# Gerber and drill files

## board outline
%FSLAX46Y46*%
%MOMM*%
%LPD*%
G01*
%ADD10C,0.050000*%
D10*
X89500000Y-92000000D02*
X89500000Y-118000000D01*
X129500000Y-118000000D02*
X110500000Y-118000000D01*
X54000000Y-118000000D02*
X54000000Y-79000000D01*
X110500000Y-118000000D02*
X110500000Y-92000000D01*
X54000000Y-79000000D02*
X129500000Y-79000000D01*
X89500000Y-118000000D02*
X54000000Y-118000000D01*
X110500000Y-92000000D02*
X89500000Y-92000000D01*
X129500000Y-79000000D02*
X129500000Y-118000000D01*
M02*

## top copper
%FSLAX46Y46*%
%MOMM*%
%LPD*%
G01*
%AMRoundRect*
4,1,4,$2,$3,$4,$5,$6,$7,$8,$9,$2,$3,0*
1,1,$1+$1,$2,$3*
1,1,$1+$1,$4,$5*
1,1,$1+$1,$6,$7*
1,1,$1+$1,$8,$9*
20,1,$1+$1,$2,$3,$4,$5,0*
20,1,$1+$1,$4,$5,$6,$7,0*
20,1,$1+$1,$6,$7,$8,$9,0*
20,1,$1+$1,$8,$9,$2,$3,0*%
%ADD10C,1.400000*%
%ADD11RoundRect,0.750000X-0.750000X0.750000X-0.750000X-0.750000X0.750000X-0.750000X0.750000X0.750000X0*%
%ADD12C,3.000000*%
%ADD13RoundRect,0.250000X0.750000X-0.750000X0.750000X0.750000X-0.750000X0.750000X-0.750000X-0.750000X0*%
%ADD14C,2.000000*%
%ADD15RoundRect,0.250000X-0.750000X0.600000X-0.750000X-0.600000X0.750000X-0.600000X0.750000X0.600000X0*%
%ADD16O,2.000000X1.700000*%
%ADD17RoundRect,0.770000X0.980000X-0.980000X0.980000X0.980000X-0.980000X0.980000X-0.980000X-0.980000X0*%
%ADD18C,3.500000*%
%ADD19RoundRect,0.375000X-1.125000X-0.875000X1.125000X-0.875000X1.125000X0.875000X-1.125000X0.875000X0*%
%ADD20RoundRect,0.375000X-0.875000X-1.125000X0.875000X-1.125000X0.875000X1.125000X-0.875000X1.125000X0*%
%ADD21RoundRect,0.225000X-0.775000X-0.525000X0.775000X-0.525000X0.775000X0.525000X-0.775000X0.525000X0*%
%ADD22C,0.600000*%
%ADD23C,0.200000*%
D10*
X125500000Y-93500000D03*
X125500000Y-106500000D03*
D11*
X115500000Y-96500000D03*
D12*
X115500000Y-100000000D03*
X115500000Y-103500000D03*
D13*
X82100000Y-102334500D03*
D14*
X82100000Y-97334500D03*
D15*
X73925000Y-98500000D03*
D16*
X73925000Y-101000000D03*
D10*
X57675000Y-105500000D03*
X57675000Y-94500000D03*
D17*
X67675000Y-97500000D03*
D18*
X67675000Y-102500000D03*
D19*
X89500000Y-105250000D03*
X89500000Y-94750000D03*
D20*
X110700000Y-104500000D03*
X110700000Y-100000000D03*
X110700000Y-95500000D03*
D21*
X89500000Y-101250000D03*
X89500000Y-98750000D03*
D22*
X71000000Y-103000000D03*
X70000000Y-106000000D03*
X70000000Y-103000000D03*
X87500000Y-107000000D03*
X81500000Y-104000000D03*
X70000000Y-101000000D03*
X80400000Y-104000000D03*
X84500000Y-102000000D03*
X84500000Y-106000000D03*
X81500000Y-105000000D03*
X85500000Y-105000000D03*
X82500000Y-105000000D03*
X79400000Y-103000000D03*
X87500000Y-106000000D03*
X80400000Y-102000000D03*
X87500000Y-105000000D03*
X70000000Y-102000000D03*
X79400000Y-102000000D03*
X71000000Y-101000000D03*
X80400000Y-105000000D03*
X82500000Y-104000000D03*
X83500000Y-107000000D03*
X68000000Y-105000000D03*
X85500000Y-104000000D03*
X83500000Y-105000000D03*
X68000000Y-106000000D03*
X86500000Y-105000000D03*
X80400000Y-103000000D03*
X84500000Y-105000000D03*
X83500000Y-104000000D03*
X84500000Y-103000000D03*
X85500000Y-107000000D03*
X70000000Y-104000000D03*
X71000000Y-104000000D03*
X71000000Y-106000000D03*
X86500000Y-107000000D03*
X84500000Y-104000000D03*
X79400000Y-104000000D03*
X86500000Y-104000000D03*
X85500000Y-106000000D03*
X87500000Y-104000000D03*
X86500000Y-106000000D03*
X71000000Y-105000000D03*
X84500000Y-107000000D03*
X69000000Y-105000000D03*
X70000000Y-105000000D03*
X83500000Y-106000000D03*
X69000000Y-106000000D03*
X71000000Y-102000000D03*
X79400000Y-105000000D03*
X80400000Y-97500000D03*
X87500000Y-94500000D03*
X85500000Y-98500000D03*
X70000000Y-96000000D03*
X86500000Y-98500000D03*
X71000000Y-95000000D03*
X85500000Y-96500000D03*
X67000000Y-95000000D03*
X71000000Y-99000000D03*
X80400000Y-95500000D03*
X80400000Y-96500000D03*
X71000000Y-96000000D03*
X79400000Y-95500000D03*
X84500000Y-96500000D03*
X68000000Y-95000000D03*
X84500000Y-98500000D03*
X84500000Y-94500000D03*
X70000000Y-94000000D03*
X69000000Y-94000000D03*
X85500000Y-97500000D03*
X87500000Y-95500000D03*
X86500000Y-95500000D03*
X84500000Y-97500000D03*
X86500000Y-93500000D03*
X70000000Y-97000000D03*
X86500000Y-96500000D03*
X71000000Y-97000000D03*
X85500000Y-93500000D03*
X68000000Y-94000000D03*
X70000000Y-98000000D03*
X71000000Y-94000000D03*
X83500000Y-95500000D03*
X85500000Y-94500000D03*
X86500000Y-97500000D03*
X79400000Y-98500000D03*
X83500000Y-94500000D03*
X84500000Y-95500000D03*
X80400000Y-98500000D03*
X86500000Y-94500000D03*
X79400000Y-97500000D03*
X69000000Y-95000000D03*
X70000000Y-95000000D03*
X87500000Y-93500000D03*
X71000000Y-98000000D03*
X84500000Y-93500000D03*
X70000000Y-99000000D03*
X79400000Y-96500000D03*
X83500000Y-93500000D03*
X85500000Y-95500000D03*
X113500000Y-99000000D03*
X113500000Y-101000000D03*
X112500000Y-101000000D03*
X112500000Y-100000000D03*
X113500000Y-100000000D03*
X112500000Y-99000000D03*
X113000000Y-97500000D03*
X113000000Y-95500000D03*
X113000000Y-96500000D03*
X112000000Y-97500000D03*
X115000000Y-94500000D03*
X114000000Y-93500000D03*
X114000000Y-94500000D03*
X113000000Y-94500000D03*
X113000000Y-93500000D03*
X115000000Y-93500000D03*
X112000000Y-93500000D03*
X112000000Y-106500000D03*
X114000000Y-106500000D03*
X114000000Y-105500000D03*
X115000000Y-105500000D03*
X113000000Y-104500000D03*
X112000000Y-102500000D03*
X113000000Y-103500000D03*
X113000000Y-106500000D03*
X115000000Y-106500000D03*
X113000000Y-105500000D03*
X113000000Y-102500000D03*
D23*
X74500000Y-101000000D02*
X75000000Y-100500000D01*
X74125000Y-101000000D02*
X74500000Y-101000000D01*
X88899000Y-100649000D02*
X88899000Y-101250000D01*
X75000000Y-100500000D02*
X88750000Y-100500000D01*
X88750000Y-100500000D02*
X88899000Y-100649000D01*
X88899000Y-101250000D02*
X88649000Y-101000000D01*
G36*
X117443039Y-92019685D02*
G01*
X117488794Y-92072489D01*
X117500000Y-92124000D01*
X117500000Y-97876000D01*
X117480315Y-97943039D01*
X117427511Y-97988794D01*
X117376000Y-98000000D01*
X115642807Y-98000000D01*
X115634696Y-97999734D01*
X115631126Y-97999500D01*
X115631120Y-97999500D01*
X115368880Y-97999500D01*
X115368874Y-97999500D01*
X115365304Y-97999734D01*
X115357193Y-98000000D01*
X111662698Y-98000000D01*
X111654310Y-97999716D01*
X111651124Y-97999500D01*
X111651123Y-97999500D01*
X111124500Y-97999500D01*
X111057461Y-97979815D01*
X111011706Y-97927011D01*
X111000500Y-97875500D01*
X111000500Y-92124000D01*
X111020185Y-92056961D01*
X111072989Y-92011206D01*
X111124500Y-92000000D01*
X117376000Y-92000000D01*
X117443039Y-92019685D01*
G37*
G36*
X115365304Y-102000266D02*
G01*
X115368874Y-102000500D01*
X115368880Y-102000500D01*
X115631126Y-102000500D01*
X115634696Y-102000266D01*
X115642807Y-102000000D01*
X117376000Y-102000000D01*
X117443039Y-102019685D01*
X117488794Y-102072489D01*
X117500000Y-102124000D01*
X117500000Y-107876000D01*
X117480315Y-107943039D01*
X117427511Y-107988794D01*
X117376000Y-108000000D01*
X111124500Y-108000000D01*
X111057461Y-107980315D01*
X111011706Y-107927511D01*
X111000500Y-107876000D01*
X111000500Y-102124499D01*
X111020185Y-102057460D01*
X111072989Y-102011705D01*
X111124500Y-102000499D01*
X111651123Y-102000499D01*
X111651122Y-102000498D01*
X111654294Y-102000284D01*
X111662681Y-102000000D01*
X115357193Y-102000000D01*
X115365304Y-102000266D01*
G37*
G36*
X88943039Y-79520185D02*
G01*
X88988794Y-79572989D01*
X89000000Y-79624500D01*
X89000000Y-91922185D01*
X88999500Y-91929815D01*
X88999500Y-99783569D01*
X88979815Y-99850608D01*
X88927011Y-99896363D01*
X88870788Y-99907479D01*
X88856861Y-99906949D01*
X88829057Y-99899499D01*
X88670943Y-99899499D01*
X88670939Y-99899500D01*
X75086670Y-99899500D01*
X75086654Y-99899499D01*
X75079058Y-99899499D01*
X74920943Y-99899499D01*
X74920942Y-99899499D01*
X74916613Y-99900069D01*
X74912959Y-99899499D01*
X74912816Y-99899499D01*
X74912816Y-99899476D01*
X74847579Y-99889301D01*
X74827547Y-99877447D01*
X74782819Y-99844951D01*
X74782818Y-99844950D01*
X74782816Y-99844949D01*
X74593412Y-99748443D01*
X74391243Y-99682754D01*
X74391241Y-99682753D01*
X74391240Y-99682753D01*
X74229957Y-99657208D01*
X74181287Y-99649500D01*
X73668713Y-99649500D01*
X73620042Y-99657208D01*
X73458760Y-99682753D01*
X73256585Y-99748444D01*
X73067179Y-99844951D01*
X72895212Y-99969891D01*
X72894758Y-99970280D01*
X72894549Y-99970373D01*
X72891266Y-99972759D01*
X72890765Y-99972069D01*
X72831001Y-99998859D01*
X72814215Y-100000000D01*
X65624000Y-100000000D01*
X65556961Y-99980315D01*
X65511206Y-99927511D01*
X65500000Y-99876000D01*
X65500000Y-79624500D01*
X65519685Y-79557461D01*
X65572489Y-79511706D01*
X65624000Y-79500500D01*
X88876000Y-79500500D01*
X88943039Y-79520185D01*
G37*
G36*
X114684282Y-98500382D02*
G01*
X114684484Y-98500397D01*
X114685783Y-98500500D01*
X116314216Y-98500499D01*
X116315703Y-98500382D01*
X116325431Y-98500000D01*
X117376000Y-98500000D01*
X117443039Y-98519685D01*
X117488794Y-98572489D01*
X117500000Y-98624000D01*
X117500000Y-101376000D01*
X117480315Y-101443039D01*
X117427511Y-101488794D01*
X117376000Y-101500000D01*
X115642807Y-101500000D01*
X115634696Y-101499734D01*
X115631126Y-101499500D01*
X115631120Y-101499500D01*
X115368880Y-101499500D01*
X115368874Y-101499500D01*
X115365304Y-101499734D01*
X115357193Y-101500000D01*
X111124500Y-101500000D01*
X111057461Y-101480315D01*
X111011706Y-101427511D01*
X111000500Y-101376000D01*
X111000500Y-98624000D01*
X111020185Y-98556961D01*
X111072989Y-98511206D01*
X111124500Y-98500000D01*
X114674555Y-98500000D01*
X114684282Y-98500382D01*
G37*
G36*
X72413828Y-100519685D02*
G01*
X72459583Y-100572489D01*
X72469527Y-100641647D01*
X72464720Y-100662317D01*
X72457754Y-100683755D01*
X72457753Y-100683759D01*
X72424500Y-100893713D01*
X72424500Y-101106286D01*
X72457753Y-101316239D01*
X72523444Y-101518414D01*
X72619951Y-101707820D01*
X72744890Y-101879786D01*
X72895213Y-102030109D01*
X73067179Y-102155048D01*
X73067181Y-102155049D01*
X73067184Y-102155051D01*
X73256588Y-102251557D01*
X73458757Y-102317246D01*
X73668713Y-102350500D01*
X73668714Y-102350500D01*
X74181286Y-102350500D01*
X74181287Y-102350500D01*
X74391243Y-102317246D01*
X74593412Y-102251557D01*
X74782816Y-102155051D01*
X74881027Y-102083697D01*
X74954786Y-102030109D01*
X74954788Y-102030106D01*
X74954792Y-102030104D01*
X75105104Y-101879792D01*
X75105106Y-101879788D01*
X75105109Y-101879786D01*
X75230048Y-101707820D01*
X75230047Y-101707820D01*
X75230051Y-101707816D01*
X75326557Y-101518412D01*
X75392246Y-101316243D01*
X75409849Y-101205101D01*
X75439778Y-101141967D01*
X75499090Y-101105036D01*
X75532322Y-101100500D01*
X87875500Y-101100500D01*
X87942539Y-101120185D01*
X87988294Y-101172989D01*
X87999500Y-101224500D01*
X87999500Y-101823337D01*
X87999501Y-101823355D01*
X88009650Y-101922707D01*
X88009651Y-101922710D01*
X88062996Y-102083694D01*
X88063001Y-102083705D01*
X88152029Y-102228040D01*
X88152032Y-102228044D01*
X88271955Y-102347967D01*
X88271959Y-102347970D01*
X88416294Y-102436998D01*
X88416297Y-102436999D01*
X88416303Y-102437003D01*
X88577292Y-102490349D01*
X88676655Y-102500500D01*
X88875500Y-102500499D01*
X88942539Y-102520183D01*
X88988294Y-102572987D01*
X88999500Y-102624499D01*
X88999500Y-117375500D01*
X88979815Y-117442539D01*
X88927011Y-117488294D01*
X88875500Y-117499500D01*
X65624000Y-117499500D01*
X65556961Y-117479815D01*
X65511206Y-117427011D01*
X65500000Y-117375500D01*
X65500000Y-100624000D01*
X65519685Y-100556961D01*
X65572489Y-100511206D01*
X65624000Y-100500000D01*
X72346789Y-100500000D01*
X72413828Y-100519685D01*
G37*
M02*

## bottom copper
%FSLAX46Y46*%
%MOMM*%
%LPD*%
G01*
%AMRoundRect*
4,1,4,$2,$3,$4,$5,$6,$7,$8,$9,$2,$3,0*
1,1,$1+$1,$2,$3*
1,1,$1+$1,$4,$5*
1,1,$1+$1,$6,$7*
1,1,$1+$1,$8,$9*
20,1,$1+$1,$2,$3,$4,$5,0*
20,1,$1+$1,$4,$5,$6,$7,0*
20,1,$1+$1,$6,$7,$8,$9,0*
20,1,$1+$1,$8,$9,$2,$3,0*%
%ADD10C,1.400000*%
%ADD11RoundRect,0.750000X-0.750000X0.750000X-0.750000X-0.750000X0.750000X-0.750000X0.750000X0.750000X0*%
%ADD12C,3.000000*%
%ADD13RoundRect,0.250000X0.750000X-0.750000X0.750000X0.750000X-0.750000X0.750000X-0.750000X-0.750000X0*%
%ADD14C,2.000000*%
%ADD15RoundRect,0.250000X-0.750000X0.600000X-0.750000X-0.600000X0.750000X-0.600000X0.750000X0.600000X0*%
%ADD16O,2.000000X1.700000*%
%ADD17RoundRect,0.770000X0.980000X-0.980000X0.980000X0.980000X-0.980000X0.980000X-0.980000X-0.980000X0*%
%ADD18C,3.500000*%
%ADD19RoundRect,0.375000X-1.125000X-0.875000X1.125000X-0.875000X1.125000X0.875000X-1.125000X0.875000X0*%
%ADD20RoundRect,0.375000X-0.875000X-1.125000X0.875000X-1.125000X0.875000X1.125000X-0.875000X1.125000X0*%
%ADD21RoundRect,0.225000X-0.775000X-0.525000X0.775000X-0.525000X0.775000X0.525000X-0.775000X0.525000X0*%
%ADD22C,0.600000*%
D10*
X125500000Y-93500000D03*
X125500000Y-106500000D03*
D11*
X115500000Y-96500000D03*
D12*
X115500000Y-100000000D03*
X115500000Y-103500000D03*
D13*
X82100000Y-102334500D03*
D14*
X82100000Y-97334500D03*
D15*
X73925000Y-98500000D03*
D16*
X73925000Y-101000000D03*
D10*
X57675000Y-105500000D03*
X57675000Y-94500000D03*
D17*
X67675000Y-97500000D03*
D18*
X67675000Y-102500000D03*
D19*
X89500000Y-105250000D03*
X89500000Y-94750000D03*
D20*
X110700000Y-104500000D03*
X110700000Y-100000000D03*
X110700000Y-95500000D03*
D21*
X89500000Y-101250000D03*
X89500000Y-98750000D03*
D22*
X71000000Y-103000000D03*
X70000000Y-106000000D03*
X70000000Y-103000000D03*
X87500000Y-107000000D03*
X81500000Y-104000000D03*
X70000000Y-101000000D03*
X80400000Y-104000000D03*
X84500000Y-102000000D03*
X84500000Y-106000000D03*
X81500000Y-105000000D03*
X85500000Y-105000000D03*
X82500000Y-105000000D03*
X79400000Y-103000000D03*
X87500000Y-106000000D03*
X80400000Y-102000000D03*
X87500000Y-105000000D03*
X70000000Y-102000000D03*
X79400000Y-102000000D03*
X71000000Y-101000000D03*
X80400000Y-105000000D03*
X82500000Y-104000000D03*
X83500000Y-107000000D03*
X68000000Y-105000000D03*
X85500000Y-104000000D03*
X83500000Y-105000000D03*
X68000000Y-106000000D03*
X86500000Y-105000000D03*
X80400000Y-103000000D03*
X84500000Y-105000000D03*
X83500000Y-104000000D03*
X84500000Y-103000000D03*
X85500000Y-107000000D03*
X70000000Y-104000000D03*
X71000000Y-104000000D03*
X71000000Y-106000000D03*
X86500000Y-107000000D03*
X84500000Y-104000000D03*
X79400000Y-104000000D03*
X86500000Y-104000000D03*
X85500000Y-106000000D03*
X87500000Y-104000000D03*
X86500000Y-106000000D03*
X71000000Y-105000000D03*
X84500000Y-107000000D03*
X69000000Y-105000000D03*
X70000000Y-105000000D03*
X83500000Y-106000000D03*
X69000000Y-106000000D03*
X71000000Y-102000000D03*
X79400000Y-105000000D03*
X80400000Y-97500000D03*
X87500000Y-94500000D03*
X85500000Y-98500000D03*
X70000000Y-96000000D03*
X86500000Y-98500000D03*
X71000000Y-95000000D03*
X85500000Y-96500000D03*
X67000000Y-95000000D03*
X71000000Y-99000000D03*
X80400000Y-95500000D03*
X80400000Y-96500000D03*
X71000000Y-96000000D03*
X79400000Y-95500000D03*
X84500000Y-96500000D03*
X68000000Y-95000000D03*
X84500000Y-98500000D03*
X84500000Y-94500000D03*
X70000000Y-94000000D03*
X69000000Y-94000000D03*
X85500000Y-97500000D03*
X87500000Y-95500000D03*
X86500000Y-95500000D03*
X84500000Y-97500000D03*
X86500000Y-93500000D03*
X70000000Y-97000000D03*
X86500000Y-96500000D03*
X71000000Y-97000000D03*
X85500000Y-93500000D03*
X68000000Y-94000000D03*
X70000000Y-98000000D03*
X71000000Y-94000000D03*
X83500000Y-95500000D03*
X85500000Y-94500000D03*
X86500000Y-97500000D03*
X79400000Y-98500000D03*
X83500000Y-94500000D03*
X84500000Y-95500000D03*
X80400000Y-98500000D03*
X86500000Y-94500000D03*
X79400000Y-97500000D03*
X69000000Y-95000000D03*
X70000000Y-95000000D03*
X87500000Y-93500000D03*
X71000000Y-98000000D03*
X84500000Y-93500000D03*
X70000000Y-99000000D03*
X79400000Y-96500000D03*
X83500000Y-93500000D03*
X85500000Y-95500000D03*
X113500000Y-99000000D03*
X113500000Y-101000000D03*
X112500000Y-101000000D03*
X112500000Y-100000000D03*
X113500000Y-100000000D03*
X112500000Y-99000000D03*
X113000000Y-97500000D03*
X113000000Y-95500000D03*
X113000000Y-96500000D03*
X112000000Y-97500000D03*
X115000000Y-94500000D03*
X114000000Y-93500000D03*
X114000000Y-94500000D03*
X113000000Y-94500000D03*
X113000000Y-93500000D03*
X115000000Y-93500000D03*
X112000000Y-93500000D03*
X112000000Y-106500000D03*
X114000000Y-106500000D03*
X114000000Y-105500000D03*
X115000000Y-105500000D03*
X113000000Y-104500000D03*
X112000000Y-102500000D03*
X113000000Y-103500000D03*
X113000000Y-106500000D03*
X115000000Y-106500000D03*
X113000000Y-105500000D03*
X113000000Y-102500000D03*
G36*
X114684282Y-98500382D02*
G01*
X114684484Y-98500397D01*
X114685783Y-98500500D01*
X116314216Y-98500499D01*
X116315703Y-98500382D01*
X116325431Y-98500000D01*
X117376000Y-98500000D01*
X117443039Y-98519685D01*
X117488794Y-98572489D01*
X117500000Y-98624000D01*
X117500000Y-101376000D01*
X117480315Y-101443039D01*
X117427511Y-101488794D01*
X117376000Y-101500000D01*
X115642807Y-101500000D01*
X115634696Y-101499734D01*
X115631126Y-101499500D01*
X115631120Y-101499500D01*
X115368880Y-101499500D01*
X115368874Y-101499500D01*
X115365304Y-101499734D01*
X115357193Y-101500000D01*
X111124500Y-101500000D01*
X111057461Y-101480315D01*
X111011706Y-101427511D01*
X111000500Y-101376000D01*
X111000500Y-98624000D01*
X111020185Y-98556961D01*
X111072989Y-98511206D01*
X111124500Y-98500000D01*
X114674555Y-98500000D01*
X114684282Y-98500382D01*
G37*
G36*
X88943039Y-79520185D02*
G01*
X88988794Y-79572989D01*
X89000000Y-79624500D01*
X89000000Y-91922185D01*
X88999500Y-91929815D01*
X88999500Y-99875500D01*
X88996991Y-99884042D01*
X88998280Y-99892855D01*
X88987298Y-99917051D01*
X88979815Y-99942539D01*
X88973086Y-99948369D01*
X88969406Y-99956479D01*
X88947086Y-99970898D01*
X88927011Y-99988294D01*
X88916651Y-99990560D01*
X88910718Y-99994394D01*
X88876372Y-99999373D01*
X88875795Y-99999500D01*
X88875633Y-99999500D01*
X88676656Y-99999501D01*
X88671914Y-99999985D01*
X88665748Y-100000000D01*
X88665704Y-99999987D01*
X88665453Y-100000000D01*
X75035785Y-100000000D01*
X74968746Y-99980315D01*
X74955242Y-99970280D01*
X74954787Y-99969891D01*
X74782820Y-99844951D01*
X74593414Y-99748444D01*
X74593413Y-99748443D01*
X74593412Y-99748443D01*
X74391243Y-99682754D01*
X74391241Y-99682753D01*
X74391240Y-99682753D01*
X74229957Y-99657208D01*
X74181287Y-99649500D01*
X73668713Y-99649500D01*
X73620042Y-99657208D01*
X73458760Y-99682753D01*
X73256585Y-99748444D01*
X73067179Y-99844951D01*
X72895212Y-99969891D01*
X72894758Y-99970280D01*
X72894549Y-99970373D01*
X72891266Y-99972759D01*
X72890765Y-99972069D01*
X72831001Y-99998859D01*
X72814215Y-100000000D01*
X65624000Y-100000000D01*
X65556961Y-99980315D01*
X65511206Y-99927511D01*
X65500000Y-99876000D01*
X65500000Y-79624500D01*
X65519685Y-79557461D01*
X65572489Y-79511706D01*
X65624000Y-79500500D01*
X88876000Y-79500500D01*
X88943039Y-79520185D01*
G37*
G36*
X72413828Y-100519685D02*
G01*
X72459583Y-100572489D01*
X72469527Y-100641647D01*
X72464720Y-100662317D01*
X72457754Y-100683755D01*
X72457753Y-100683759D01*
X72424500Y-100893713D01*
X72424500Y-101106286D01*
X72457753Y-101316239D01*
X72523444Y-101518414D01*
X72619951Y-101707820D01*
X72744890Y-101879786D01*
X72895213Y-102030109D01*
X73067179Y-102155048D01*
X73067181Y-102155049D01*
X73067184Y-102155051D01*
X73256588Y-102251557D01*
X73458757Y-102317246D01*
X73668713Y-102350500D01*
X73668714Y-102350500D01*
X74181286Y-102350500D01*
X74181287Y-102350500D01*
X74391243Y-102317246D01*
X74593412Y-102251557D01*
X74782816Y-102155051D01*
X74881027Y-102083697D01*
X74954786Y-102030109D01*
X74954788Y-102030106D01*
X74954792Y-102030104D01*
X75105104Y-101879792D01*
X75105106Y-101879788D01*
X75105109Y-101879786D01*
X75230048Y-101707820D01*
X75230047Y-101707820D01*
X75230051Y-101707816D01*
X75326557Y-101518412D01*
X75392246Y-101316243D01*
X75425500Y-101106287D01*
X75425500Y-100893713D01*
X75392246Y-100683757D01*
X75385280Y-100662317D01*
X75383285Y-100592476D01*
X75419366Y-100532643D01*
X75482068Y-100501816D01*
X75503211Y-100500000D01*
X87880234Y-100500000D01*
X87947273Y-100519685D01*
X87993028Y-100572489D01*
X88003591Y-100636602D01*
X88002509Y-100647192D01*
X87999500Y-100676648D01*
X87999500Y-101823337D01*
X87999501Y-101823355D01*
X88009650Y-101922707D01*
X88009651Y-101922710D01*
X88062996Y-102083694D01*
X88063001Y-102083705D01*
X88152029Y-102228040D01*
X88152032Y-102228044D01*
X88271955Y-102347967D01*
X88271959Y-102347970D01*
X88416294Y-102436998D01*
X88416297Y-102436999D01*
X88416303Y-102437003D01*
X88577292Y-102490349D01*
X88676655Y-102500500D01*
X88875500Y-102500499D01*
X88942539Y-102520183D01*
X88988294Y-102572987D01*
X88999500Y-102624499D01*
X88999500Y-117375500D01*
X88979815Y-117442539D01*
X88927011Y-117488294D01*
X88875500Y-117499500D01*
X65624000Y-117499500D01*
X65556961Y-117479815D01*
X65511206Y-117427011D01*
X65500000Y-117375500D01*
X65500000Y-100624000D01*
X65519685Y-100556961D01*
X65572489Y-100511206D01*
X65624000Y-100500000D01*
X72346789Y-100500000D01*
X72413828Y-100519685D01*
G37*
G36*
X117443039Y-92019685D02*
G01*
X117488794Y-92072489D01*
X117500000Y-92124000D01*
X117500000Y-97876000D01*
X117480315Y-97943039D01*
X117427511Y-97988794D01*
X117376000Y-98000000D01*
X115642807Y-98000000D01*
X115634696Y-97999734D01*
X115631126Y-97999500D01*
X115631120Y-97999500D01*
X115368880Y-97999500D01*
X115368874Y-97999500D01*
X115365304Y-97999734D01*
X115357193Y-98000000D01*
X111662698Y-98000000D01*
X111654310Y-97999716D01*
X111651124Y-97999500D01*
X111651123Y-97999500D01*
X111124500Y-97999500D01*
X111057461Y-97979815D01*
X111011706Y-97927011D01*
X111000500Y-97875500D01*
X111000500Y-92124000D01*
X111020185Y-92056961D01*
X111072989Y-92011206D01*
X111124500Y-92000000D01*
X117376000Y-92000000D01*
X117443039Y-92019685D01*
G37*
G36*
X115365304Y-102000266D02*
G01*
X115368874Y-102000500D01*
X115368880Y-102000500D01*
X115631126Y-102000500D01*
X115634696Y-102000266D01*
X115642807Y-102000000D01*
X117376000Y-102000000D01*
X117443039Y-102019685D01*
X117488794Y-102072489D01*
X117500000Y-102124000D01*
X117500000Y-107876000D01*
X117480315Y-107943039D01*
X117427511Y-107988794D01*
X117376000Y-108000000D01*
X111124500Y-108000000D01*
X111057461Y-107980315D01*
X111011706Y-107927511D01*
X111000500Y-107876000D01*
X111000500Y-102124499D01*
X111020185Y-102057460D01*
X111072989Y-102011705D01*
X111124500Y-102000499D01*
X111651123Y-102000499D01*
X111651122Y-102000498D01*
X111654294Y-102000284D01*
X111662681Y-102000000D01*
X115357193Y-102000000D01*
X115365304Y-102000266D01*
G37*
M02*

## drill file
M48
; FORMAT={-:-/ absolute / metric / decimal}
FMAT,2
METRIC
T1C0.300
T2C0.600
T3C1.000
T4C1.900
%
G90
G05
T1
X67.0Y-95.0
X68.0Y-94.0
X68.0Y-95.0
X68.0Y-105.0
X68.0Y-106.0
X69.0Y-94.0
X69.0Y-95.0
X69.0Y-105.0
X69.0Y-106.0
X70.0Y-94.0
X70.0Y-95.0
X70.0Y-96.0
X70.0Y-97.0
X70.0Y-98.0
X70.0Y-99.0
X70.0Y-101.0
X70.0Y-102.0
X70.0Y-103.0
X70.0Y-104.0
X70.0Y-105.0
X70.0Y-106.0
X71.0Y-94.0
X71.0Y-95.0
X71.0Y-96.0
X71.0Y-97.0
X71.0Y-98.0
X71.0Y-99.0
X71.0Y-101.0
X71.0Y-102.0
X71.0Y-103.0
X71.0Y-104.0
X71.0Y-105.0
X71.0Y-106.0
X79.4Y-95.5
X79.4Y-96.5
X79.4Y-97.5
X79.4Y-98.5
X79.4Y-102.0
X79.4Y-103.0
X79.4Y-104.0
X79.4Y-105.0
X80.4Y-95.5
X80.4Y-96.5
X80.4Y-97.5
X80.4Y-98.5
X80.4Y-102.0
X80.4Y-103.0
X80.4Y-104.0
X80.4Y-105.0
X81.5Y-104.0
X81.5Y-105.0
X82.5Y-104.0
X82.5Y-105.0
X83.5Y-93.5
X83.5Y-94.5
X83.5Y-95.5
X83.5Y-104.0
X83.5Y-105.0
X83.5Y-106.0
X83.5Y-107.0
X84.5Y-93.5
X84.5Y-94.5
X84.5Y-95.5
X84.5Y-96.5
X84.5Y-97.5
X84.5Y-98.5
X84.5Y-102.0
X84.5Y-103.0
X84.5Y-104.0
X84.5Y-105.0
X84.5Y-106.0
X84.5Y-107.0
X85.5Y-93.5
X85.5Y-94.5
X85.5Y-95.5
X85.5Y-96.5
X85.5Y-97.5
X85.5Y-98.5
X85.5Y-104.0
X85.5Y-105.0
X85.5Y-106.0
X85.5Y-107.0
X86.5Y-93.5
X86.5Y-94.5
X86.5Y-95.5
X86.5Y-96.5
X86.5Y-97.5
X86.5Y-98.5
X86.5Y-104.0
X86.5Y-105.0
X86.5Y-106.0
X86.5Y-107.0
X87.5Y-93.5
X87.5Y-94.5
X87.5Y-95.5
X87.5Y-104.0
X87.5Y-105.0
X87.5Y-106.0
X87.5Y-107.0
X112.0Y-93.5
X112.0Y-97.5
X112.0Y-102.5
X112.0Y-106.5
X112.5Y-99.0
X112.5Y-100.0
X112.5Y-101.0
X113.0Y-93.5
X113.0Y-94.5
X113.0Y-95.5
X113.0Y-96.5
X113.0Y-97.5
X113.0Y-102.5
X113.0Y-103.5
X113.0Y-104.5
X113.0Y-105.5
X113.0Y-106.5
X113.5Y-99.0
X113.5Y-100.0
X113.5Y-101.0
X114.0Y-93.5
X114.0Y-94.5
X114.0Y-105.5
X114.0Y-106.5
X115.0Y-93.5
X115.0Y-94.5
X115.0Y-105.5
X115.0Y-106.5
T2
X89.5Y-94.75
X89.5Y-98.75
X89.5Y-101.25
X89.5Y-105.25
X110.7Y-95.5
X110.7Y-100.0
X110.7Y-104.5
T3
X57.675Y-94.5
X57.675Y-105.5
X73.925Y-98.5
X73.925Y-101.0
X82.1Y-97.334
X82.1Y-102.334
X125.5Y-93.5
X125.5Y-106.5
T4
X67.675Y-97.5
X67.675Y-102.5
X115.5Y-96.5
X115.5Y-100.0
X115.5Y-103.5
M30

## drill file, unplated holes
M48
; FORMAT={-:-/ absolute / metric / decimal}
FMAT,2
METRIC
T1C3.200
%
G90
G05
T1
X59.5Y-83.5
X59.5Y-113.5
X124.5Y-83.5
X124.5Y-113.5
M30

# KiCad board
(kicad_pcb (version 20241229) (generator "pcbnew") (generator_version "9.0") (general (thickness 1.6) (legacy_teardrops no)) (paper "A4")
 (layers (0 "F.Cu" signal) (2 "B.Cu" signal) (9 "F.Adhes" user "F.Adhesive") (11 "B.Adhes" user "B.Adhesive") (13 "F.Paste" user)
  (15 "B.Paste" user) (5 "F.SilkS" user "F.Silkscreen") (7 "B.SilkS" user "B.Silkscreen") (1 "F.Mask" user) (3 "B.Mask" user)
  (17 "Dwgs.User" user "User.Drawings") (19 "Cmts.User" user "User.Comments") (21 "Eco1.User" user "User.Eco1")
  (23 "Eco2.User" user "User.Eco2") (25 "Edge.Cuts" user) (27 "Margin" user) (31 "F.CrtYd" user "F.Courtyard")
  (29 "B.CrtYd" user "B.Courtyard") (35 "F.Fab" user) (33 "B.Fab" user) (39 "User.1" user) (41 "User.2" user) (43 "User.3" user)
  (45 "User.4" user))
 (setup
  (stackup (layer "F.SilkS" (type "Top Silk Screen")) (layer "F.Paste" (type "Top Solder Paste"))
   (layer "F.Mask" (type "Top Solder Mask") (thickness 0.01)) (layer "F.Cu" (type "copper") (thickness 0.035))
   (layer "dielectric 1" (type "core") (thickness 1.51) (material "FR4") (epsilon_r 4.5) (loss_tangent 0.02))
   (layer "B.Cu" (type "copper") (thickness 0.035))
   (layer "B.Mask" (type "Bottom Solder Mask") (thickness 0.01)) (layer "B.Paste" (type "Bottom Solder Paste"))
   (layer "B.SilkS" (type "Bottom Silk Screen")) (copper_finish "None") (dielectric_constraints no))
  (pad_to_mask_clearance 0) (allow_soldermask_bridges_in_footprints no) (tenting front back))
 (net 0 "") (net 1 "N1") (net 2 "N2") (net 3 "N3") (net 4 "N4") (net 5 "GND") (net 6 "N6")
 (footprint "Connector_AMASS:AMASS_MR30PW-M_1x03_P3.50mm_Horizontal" (layer "F.Cu") (at 115.5 96.5 -90)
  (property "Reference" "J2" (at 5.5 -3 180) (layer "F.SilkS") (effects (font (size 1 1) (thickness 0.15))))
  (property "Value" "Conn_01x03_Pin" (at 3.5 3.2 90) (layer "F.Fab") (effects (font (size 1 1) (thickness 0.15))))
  (pad "" thru_hole circle (at -3 -10 270) (size 1.4 1.4) (drill 1) (layers "*.Cu" "*.Mask") (remove_unused_layers no))
  (pad "" thru_hole circle (at 10 -10 270) (size 1.4 1.4) (drill 1) (layers "*.Cu" "*.Mask") (remove_unused_layers no))
  (pad "1" thru_hole roundrect (at 0 0 270) (size 3 3) (drill 1.9) (layers "*.Cu" "*.Mask") (remove_unused_layers no)
   (roundrect_rratio 0.25) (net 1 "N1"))
  (pad "2" thru_hole circle (at 3.5 0 270) (size 3 3) (drill 1.9) (layers "*.Cu" "*.Mask") (remove_unused_layers no) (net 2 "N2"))
  (pad "3" thru_hole circle (at 7 0 270) (size 3 3) (drill 1.9) (layers "*.Cu" "*.Mask") (remove_unused_layers no) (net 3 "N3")))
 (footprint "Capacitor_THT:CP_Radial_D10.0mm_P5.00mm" (layer "F.Cu") (at 82.1 102.3345 90)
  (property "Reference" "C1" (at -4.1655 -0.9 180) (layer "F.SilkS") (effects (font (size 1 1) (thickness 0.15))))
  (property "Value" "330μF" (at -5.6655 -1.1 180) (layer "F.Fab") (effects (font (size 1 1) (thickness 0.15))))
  (pad "1" thru_hole roundrect (at 0 0 90) (size 2 2) (drill 1) (layers "*.Cu" "*.Mask") (remove_unused_layers no) (roundrect_rratio 0.125)
   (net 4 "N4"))
  (pad "2" thru_hole circle (at 5 0 90) (size 2 2) (drill 1) (layers "*.Cu" "*.Mask") (remove_unused_layers no) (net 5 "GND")))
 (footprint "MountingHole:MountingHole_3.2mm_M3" (layer "F.Cu") (at 59.5 83.5)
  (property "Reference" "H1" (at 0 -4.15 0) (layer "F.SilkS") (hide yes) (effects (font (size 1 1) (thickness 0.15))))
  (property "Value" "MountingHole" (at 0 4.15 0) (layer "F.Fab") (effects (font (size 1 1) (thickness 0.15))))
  (pad "" np_thru_hole circle (at 0 0) (size 3.2 3.2) (drill 3.2) (layers "*.Cu" "*.Mask")))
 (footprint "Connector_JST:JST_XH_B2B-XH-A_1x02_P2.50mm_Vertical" (layer "F.Cu") (at 73.925 98.5 -90)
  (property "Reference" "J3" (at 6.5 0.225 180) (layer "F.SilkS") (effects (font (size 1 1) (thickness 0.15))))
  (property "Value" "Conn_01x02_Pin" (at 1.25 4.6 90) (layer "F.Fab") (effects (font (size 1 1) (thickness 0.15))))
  (pad "1" thru_hole roundrect (at 0 0 270) (size 1.7 2) (drill 1) (layers "*.Cu" "*.Mask") (remove_unused_layers no)
   (roundrect_rratio 0.147059) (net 5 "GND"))
  (pad "2" thru_hole oval (at 2.5 0 270) (size 1.7 2) (drill 1) (layers "*.Cu" "*.Mask") (remove_unused_layers no) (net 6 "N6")))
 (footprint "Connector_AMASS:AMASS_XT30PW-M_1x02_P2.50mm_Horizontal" (layer "F.Cu") (at 67.675 97.5 90)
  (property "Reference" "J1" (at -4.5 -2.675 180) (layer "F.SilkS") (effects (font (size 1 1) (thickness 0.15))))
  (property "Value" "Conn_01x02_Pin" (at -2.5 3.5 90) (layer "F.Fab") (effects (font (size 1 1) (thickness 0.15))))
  (pad "" thru_hole circle (at -8 -10 90) (size 1.4 1.4) (drill 1) (layers "*.Cu" "*.Mask") (remove_unused_layers no))
  (pad "" thru_hole circle (at 3 -10 90) (size 1.4 1.4) (drill 1) (layers "*.Cu" "*.Mask") (remove_unused_layers no))
  (pad "1" thru_hole roundrect (at 0 0 90) (size 3.5 3.5) (drill 1.9) (layers "*.Cu" "*.Mask") (remove_unused_layers no)
   (roundrect_rratio 0.22) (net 5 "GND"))
  (pad "2" thru_hole circle (at -5 0 90) (size 3.5 3.5) (drill 1.9) (layers "*.Cu" "*.Mask") (remove_unused_layers no) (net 4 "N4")))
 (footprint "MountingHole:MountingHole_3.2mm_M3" (layer "F.Cu") (at 124.5 113.5)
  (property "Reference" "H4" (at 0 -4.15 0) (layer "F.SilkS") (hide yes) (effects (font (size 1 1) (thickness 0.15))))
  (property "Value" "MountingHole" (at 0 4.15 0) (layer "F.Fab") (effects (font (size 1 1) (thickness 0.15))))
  (pad "" np_thru_hole circle (at 0 0) (size 3.2 3.2) (drill 3.2) (layers "*.Cu" "*.Mask")))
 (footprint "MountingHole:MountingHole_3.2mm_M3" (layer "F.Cu") (at 124.5 83.5)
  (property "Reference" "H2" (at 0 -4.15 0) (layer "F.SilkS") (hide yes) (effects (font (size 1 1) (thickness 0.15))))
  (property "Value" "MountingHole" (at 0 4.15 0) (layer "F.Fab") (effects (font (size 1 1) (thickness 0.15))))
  (pad "" np_thru_hole circle (at 0 0) (size 3.2 3.2) (drill 3.2) (layers "*.Cu" "*.Mask")))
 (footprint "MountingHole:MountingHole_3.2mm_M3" (layer "F.Cu") (at 59.5 113.5)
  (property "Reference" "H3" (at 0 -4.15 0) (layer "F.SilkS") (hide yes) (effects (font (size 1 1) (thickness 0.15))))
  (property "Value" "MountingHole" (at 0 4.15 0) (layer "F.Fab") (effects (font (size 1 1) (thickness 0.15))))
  (pad "" np_thru_hole circle (at 0 0) (size 3.2 3.2) (drill 3.2) (layers "*.Cu" "*.Mask")))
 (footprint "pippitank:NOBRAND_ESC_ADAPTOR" (layer "B.Cu") (at 100 100)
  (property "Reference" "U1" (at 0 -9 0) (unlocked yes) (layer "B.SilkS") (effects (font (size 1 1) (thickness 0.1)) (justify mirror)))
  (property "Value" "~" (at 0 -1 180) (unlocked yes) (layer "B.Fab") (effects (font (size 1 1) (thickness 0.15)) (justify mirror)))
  (pad "1" thru_hole roundrect (at -10.5 5.25) (size 3 2.5) (drill 0.6) (layers "*.Cu" "*.Mask") (remove_unused_layers no)
   (roundrect_rratio 0.15) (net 4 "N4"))
  (pad "2" thru_hole roundrect (at -10.5 -5.25) (size 3 2.5) (drill 0.6) (layers "*.Cu" "*.Mask") (remove_unused_layers no)
   (roundrect_rratio 0.15) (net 5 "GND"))
  (pad "3" thru_hole roundrect (at 10.7 4.5) (size 2.5 3) (drill 0.6) (layers "*.Cu" "*.Mask") (remove_unused_layers no)
   (roundrect_rratio 0.15) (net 3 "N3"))
  (pad "4" thru_hole roundrect (at 10.7 0) (size 2.5 3) (drill 0.6) (layers "*.Cu" "*.Mask") (remove_unused_layers no)
   (roundrect_rratio 0.15) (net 2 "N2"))
  (pad "5" thru_hole roundrect (at 10.7 -4.5) (size 2.5 3) (drill 0.6) (layers "*.Cu" "*.Mask") (remove_unused_layers no)
   (roundrect_rratio 0.15) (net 1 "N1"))
  (pad "6" thru_hole roundrect (at -10.5 1.25) (size 2 1.5) (drill 0.6) (layers "*.Cu" "*.Mask") (remove_unused_layers no)
   (roundrect_rratio 0.15) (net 6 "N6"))
  (pad "7" thru_hole roundrect (at -10.5 -1.25) (size 2 1.5) (drill 0.6) (layers "*.Cu" "*.Mask") (remove_unused_layers no)
   (roundrect_rratio 0.15) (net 5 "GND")))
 (gr_line (start 89.5 92) (end 89.5 118) (stroke (width 0.05) (type default)) (layer "Edge.Cuts"))
 (gr_line (start 129.5 118) (end 110.5 118) (stroke (width 0.05) (type solid)) (layer "Edge.Cuts"))
 (gr_line (start 54 118) (end 54 79) (stroke (width 0.05) (type solid)) (layer "Edge.Cuts"))
 (gr_line (start 110.5 118) (end 110.5 92) (stroke (width 0.05) (type default)) (layer "Edge.Cuts"))
 (gr_line (start 54 79) (end 129.5 79) (stroke (width 0.05) (type solid)) (layer "Edge.Cuts"))
 (gr_line (start 89.5 118) (end 54 118) (stroke (width 0.05) (type solid)) (layer "Edge.Cuts"))
 (gr_line (start 110.5 92) (end 89.5 92) (stroke (width 0.05) (type default)) (layer "Edge.Cuts"))
 (gr_line (start 129.5 79) (end 129.5 118) (stroke (width 0.05) (type default)) (layer "Edge.Cuts"))
 (via (at 71 103) (size 0.6) (drill 0.3) (layers "F.Cu" "B.Cu") (free yes) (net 4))
 (via (at 70 106) (size 0.6) (drill 0.3) (layers "F.Cu" "B.Cu") (free yes) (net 4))
 (via (at 70 103) (size 0.6) (drill 0.3) (layers "F.Cu" "B.Cu") (free yes) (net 4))
 (via (at 87.5 107) (size 0.6) (drill 0.3) (layers "F.Cu" "B.Cu") (free yes) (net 4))
 (via (at 81.5 104) (size 0.6) (drill 0.3) (layers "F.Cu" "B.Cu") (free yes) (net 4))
 (via (at 70 101) (size 0.6) (drill 0.3) (layers "F.Cu" "B.Cu") (free yes) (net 4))
 (via (at 80.4 104) (size 0.6) (drill 0.3) (layers "F.Cu" "B.Cu") (free yes) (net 4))
 (via (at 84.5 102) (size 0.6) (drill 0.3) (layers "F.Cu" "B.Cu") (free yes) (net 4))
 (via (at 84.5 106) (size 0.6) (drill 0.3) (layers "F.Cu" "B.Cu") (free yes) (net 4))
 (via (at 81.5 105) (size 0.6) (drill 0.3) (layers "F.Cu" "B.Cu") (free yes) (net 4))
 (via (at 85.5 105) (size 0.6) (drill 0.3) (layers "F.Cu" "B.Cu") (free yes) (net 4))
 (via (at 82.5 105) (size 0.6) (drill 0.3) (layers "F.Cu" "B.Cu") (free yes) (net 4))
 (via (at 79.4 103) (size 0.6) (drill 0.3) (layers "F.Cu" "B.Cu") (free yes) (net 4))
 (via (at 87.5 106) (size 0.6) (drill 0.3) (layers "F.Cu" "B.Cu") (free yes) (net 4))
 (via (at 80.4 102) (size 0.6) (drill 0.3) (layers "F.Cu" "B.Cu") (free yes) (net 4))
 (via (at 87.5 105) (size 0.6) (drill 0.3) (layers "F.Cu" "B.Cu") (free yes) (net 4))
 (via (at 70 102) (size 0.6) (drill 0.3) (layers "F.Cu" "B.Cu") (free yes) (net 4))
 (via (at 79.4 102) (size 0.6) (drill 0.3) (layers "F.Cu" "B.Cu") (free yes) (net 4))
 (via (at 71 101) (size 0.6) (drill 0.3) (layers "F.Cu" "B.Cu") (free yes) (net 4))
 (via (at 80.4 105) (size 0.6) (drill 0.3) (layers "F.Cu" "B.Cu") (free yes) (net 4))
 (via (at 82.5 104) (size 0.6) (drill 0.3) (layers "F.Cu" "B.Cu") (free yes) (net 4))
 (via (at 83.5 107) (size 0.6) (drill 0.3) (layers "F.Cu" "B.Cu") (free yes) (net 4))
 (via (at 68 105) (size 0.6) (drill 0.3) (layers "F.Cu" "B.Cu") (free yes) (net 4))
 (via (at 85.5 104) (size 0.6) (drill 0.3) (layers "F.Cu" "B.Cu") (free yes) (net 4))
 (via (at 83.5 105) (size 0.6) (drill 0.3) (layers "F.Cu" "B.Cu") (free yes) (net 4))
 (via (at 68 106) (size 0.6) (drill 0.3) (layers "F.Cu" "B.Cu") (free yes) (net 4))
 (via (at 86.5 105) (size 0.6) (drill 0.3) (layers "F.Cu" "B.Cu") (free yes) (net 4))
 (via (at 80.4 103) (size 0.6) (drill 0.3) (layers "F.Cu" "B.Cu") (free yes) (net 4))
 (via (at 84.5 105) (size 0.6) (drill 0.3) (layers "F.Cu" "B.Cu") (free yes) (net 4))
 (via (at 83.5 104) (size 0.6) (drill 0.3) (layers "F.Cu" "B.Cu") (free yes) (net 4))
 (via (at 84.5 103) (size 0.6) (drill 0.3) (layers "F.Cu" "B.Cu") (free yes) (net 4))
 (via (at 85.5 107) (size 0.6) (drill 0.3) (layers "F.Cu" "B.Cu") (free yes) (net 4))
 (via (at 70 104) (size 0.6) (drill 0.3) (layers "F.Cu" "B.Cu") (free yes) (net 4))
 (via (at 71 104) (size 0.6) (drill 0.3) (layers "F.Cu" "B.Cu") (free yes) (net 4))
 (via (at 71 106) (size 0.6) (drill 0.3) (layers "F.Cu" "B.Cu") (free yes) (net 4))
 (via (at 86.5 107) (size 0.6) (drill 0.3) (layers "F.Cu" "B.Cu") (free yes) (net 4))
 (via (at 84.5 104) (size 0.6) (drill 0.3) (layers "F.Cu" "B.Cu") (free yes) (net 4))
 (via (at 79.4 104) (size 0.6) (drill 0.3) (layers "F.Cu" "B.Cu") (free yes) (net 4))
 (via (at 86.5 104) (size 0.6) (drill 0.3) (layers "F.Cu" "B.Cu") (free yes) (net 4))
 (via (at 85.5 106) (size 0.6) (drill 0.3) (layers "F.Cu" "B.Cu") (free yes) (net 4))
 (via (at 87.5 104) (size 0.6) (drill 0.3) (layers "F.Cu" "B.Cu") (free yes) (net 4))
 (via (at 86.5 106) (size 0.6) (drill 0.3) (layers "F.Cu" "B.Cu") (free yes) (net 4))
 (via (at 71 105) (size 0.6) (drill 0.3) (layers "F.Cu" "B.Cu") (free yes) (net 4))
 (via (at 84.5 107) (size 0.6) (drill 0.3) (layers "F.Cu" "B.Cu") (free yes) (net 4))
 (via (at 69 105) (size 0.6) (drill 0.3) (layers "F.Cu" "B.Cu") (free yes) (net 4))
 (via (at 70 105) (size 0.6) (drill 0.3) (layers "F.Cu" "B.Cu") (free yes) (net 4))
 (via (at 83.5 106) (size 0.6) (drill 0.3) (layers "F.Cu" "B.Cu") (free yes) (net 4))
 (via (at 69 106) (size 0.6) (drill 0.3) (layers "F.Cu" "B.Cu") (free yes) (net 4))
 (via (at 71 102) (size 0.6) (drill 0.3) (layers "F.Cu" "B.Cu") (free yes) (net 4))
 (via (at 79.4 105) (size 0.6) (drill 0.3) (layers "F.Cu" "B.Cu") (free yes) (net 4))
 (via (at 80.4 97.5) (size 0.6) (drill 0.3) (layers "F.Cu" "B.Cu") (free yes) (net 5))
 (via (at 87.5 94.5) (size 0.6) (drill 0.3) (layers "F.Cu" "B.Cu") (free yes) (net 5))
 (via (at 85.5 98.5) (size 0.6) (drill 0.3) (layers "F.Cu" "B.Cu") (free yes) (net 5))
 (via (at 70 96) (size 0.6) (drill 0.3) (layers "F.Cu" "B.Cu") (free yes) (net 5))
 (via (at 86.5 98.5) (size 0.6) (drill 0.3) (layers "F.Cu" "B.Cu") (free yes) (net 5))
 (via (at 71 95) (size 0.6) (drill 0.3) (layers "F.Cu" "B.Cu") (free yes) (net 5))
 (via (at 85.5 96.5) (size 0.6) (drill 0.3) (layers "F.Cu" "B.Cu") (free yes) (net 5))
 (via (at 67 95) (size 0.6) (drill 0.3) (layers "F.Cu" "B.Cu") (free yes) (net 5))
 (via (at 71 99) (size 0.6) (drill 0.3) (layers "F.Cu" "B.Cu") (free yes) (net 5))
 (via (at 80.4 95.5) (size 0.6) (drill 0.3) (layers "F.Cu" "B.Cu") (free yes) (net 5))
 (via (at 80.4 96.5) (size 0.6) (drill 0.3) (layers "F.Cu" "B.Cu") (free yes) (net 5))
 (via (at 71 96) (size 0.6) (drill 0.3) (layers "F.Cu" "B.Cu") (free yes) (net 5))
 (via (at 79.4 95.5) (size 0.6) (drill 0.3) (layers "F.Cu" "B.Cu") (free yes) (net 5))
 (via (at 84.5 96.5) (size 0.6) (drill 0.3) (layers "F.Cu" "B.Cu") (free yes) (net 5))
 (via (at 68 95) (size 0.6) (drill 0.3) (layers "F.Cu" "B.Cu") (free yes) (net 5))
 (via (at 84.5 98.5) (size 0.6) (drill 0.3) (layers "F.Cu" "B.Cu") (free yes) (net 5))
 (via (at 84.5 94.5) (size 0.6) (drill 0.3) (layers "F.Cu" "B.Cu") (free yes) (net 5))
 (via (at 70 94) (size 0.6) (drill 0.3) (layers "F.Cu" "B.Cu") (free yes) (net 5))
 (via (at 69 94) (size 0.6) (drill 0.3) (layers "F.Cu" "B.Cu") (free yes) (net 5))
 (via (at 85.5 97.5) (size 0.6) (drill 0.3) (layers "F.Cu" "B.Cu") (free yes) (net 5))
 (via (at 87.5 95.5) (size 0.6) (drill 0.3) (layers "F.Cu" "B.Cu") (free yes) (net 5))
 (via (at 86.5 95.5) (size 0.6) (drill 0.3) (layers "F.Cu" "B.Cu") (free yes) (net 5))
 (via (at 84.5 97.5) (size 0.6) (drill 0.3) (layers "F.Cu" "B.Cu") (free yes) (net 5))
 (via (at 86.5 93.5) (size 0.6) (drill 0.3) (layers "F.Cu" "B.Cu") (free yes) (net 5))
 (via (at 70 97) (size 0.6) (drill 0.3) (layers "F.Cu" "B.Cu") (free yes) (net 5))
 (via (at 86.5 96.5) (size 0.6) (drill 0.3) (layers "F.Cu" "B.Cu") (free yes) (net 5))
 (via (at 71 97) (size 0.6) (drill 0.3) (layers "F.Cu" "B.Cu") (free yes) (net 5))
 (via (at 85.5 93.5) (size 0.6) (drill 0.3) (layers "F.Cu" "B.Cu") (free yes) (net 5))
 (via (at 68 94) (size 0.6) (drill 0.3) (layers "F.Cu" "B.Cu") (free yes) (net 5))
 (via (at 70 98) (size 0.6) (drill 0.3) (layers "F.Cu" "B.Cu") (free yes) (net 5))
 (via (at 71 94) (size 0.6) (drill 0.3) (layers "F.Cu" "B.Cu") (free yes) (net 5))
 (via (at 83.5 95.5) (size 0.6) (drill 0.3) (layers "F.Cu" "B.Cu") (free yes) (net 5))
 (via (at 85.5 94.5) (size 0.6) (drill 0.3) (layers "F.Cu" "B.Cu") (free yes) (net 5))
 (via (at 86.5 97.5) (size 0.6) (drill 0.3) (layers "F.Cu" "B.Cu") (free yes) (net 5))
 (via (at 79.4 98.5) (size 0.6) (drill 0.3) (layers "F.Cu" "B.Cu") (free yes) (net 5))
 (via (at 83.5 94.5) (size 0.6) (drill 0.3) (layers "F.Cu" "B.Cu") (free yes) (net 5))
 (via (at 84.5 95.5) (size 0.6) (drill 0.3) (layers "F.Cu" "B.Cu") (free yes) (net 5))
 (via (at 80.4 98.5) (size 0.6) (drill 0.3) (layers "F.Cu" "B.Cu") (free yes) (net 5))
 (via (at 86.5 94.5) (size 0.6) (drill 0.3) (layers "F.Cu" "B.Cu") (free yes) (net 5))
 (via (at 79.4 97.5) (size 0.6) (drill 0.3) (layers "F.Cu" "B.Cu") (free yes) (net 5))
 (via (at 69 95) (size 0.6) (drill 0.3) (layers "F.Cu" "B.Cu") (free yes) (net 5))
 (via (at 70 95) (size 0.6) (drill 0.3) (layers "F.Cu" "B.Cu") (free yes) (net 5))
 (via (at 87.5 93.5) (size 0.6) (drill 0.3) (layers "F.Cu" "B.Cu") (free yes) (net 5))
 (via (at 71 98) (size 0.6) (drill 0.3) (layers "F.Cu" "B.Cu") (free yes) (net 5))
 (via (at 84.5 93.5) (size 0.6) (drill 0.3) (layers "F.Cu" "B.Cu") (free yes) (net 5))
 (via (at 70 99) (size 0.6) (drill 0.3) (layers "F.Cu" "B.Cu") (free yes) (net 5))
 (via (at 79.4 96.5) (size 0.6) (drill 0.3) (layers "F.Cu" "B.Cu") (free yes) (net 5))
 (via (at 83.5 93.5) (size 0.6) (drill 0.3) (layers "F.Cu" "B.Cu") (free yes) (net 5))
 (via (at 85.5 95.5) (size 0.6) (drill 0.3) (layers "F.Cu" "B.Cu") (free yes) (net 5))
 (via (at 113.5 99) (size 0.6) (drill 0.3) (layers "F.Cu" "B.Cu") (free yes) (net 2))
 (via (at 113.5 101) (size 0.6) (drill 0.3) (layers "F.Cu" "B.Cu") (free yes) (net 2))
 (via (at 112.5 101) (size 0.6) (drill 0.3) (layers "F.Cu" "B.Cu") (free yes) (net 2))
 (via (at 112.5 100) (size 0.6) (drill 0.3) (layers "F.Cu" "B.Cu") (free yes) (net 2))
 (via (at 113.5 100) (size 0.6) (drill 0.3) (layers "F.Cu" "B.Cu") (free yes) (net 2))
 (via (at 112.5 99) (size 0.6) (drill 0.3) (layers "F.Cu" "B.Cu") (free yes) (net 2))
 (via (at 113 97.5) (size 0.6) (drill 0.3) (layers "F.Cu" "B.Cu") (free yes) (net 1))
 (via (at 113 95.5) (size 0.6) (drill 0.3) (layers "F.Cu" "B.Cu") (free yes) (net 1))
 (via (at 113 96.5) (size 0.6) (drill 0.3) (layers "F.Cu" "B.Cu") (free yes) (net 1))
 (via (at 112 97.5) (size 0.6) (drill 0.3) (layers "F.Cu" "B.Cu") (free yes) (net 1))
 (via (at 115 94.5) (size 0.6) (drill 0.3) (layers "F.Cu" "B.Cu") (free yes) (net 1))
 (via (at 114 93.5) (size 0.6) (drill 0.3) (layers "F.Cu" "B.Cu") (free yes) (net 1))
 (via (at 114 94.5) (size 0.6) (drill 0.3) (layers "F.Cu" "B.Cu") (free yes) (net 1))
 (via (at 113 94.5) (size 0.6) (drill 0.3) (layers "F.Cu" "B.Cu") (free yes) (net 1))
 (via (at 113 93.5) (size 0.6) (drill 0.3) (layers "F.Cu" "B.Cu") (free yes) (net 1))
 (via (at 115 93.5) (size 0.6) (drill 0.3) (layers "F.Cu" "B.Cu") (free yes) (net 1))
 (via (at 112 93.5) (size 0.6) (drill 0.3) (layers "F.Cu" "B.Cu") (free yes) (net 1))
 (via (at 112 106.5) (size 0.6) (drill 0.3) (layers "F.Cu" "B.Cu") (free yes) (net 3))
 (via (at 114 106.5) (size 0.6) (drill 0.3) (layers "F.Cu" "B.Cu") (free yes) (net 3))
 (via (at 114 105.5) (size 0.6) (drill 0.3) (layers "F.Cu" "B.Cu") (free yes) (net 3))
 (via (at 115 105.5) (size 0.6) (drill 0.3) (layers "F.Cu" "B.Cu") (free yes) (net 3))
 (via (at 113 104.5) (size 0.6) (drill 0.3) (layers "F.Cu" "B.Cu") (free yes) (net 3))
 (via (at 112 102.5) (size 0.6) (drill 0.3) (layers "F.Cu" "B.Cu") (free yes) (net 3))
 (via (at 113 103.5) (size 0.6) (drill 0.3) (layers "F.Cu" "B.Cu") (free yes) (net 3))
 (via (at 113 106.5) (size 0.6) (drill 0.3) (layers "F.Cu" "B.Cu") (free yes) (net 3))
 (via (at 115 106.5) (size 0.6) (drill 0.3) (layers "F.Cu" "B.Cu") (free yes) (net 3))
 (via (at 113 105.5) (size 0.6) (drill 0.3) (layers "F.Cu" "B.Cu") (free yes) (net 3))
 (via (at 113 102.5) (size 0.6) (drill 0.3) (layers "F.Cu" "B.Cu") (free yes) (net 3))
 (segment (start 74.5 101) (end 75 100.5) (width 0.2) (layer "F.Cu") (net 6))
 (segment (start 74.125 101) (end 74.5 101) (width 0.2) (layer "F.Cu") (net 6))
 (segment (start 88.899 100.649) (end 88.899 101.25) (width 0.2) (layer "F.Cu") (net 6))
 (segment (start 75 100.5) (end 88.75 100.5) (width 0.2) (layer "F.Cu") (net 6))
 (segment (start 88.75 100.5) (end 88.899 100.649) (width 0.2) (layer "F.Cu") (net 6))
 (segment (start 88.899 101.25) (end 88.649 101) (width 0.2) (layer "F.Cu") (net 6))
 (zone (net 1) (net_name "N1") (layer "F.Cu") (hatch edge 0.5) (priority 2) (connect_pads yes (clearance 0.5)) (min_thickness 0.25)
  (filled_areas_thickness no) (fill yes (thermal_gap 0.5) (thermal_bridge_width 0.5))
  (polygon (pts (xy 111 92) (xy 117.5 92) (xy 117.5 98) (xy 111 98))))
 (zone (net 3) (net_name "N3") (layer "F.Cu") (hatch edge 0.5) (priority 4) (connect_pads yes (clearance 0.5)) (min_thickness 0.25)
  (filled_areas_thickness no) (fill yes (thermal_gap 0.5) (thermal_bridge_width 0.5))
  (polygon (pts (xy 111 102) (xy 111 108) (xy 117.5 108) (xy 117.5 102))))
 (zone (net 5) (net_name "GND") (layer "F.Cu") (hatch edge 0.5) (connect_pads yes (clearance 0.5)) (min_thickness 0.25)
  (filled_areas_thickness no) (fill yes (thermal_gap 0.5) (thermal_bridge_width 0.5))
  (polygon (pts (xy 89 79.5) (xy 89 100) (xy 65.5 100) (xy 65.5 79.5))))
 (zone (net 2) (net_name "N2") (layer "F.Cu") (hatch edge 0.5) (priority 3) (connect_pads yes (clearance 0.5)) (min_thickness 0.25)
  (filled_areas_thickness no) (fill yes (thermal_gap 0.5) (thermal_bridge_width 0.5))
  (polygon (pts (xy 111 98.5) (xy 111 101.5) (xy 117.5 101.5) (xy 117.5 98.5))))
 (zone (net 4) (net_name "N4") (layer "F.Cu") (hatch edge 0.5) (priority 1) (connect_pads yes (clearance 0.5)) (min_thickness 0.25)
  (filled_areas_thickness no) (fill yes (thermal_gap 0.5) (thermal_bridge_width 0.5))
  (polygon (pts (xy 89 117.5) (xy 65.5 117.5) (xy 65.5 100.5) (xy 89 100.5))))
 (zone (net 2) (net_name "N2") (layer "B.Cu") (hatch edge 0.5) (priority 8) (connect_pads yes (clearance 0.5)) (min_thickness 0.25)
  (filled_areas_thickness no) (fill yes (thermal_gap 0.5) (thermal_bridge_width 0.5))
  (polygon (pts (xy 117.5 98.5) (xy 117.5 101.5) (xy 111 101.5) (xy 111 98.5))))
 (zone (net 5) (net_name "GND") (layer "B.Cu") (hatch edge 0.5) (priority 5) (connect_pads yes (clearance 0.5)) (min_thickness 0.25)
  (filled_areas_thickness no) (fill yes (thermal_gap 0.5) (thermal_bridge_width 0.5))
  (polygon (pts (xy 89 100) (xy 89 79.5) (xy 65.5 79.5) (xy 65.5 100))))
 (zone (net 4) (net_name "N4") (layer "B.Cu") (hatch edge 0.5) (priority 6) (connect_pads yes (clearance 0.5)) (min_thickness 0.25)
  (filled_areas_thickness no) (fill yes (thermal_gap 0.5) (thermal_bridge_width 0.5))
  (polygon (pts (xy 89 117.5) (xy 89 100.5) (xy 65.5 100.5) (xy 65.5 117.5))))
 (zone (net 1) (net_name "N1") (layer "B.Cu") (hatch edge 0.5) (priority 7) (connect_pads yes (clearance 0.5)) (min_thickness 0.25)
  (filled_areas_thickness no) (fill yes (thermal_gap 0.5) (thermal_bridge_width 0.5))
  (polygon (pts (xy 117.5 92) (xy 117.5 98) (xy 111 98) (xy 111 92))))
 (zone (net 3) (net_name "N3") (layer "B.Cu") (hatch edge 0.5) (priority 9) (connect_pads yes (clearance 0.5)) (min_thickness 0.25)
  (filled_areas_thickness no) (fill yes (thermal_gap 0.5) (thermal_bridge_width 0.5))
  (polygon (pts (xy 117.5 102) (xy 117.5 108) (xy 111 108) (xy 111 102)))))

